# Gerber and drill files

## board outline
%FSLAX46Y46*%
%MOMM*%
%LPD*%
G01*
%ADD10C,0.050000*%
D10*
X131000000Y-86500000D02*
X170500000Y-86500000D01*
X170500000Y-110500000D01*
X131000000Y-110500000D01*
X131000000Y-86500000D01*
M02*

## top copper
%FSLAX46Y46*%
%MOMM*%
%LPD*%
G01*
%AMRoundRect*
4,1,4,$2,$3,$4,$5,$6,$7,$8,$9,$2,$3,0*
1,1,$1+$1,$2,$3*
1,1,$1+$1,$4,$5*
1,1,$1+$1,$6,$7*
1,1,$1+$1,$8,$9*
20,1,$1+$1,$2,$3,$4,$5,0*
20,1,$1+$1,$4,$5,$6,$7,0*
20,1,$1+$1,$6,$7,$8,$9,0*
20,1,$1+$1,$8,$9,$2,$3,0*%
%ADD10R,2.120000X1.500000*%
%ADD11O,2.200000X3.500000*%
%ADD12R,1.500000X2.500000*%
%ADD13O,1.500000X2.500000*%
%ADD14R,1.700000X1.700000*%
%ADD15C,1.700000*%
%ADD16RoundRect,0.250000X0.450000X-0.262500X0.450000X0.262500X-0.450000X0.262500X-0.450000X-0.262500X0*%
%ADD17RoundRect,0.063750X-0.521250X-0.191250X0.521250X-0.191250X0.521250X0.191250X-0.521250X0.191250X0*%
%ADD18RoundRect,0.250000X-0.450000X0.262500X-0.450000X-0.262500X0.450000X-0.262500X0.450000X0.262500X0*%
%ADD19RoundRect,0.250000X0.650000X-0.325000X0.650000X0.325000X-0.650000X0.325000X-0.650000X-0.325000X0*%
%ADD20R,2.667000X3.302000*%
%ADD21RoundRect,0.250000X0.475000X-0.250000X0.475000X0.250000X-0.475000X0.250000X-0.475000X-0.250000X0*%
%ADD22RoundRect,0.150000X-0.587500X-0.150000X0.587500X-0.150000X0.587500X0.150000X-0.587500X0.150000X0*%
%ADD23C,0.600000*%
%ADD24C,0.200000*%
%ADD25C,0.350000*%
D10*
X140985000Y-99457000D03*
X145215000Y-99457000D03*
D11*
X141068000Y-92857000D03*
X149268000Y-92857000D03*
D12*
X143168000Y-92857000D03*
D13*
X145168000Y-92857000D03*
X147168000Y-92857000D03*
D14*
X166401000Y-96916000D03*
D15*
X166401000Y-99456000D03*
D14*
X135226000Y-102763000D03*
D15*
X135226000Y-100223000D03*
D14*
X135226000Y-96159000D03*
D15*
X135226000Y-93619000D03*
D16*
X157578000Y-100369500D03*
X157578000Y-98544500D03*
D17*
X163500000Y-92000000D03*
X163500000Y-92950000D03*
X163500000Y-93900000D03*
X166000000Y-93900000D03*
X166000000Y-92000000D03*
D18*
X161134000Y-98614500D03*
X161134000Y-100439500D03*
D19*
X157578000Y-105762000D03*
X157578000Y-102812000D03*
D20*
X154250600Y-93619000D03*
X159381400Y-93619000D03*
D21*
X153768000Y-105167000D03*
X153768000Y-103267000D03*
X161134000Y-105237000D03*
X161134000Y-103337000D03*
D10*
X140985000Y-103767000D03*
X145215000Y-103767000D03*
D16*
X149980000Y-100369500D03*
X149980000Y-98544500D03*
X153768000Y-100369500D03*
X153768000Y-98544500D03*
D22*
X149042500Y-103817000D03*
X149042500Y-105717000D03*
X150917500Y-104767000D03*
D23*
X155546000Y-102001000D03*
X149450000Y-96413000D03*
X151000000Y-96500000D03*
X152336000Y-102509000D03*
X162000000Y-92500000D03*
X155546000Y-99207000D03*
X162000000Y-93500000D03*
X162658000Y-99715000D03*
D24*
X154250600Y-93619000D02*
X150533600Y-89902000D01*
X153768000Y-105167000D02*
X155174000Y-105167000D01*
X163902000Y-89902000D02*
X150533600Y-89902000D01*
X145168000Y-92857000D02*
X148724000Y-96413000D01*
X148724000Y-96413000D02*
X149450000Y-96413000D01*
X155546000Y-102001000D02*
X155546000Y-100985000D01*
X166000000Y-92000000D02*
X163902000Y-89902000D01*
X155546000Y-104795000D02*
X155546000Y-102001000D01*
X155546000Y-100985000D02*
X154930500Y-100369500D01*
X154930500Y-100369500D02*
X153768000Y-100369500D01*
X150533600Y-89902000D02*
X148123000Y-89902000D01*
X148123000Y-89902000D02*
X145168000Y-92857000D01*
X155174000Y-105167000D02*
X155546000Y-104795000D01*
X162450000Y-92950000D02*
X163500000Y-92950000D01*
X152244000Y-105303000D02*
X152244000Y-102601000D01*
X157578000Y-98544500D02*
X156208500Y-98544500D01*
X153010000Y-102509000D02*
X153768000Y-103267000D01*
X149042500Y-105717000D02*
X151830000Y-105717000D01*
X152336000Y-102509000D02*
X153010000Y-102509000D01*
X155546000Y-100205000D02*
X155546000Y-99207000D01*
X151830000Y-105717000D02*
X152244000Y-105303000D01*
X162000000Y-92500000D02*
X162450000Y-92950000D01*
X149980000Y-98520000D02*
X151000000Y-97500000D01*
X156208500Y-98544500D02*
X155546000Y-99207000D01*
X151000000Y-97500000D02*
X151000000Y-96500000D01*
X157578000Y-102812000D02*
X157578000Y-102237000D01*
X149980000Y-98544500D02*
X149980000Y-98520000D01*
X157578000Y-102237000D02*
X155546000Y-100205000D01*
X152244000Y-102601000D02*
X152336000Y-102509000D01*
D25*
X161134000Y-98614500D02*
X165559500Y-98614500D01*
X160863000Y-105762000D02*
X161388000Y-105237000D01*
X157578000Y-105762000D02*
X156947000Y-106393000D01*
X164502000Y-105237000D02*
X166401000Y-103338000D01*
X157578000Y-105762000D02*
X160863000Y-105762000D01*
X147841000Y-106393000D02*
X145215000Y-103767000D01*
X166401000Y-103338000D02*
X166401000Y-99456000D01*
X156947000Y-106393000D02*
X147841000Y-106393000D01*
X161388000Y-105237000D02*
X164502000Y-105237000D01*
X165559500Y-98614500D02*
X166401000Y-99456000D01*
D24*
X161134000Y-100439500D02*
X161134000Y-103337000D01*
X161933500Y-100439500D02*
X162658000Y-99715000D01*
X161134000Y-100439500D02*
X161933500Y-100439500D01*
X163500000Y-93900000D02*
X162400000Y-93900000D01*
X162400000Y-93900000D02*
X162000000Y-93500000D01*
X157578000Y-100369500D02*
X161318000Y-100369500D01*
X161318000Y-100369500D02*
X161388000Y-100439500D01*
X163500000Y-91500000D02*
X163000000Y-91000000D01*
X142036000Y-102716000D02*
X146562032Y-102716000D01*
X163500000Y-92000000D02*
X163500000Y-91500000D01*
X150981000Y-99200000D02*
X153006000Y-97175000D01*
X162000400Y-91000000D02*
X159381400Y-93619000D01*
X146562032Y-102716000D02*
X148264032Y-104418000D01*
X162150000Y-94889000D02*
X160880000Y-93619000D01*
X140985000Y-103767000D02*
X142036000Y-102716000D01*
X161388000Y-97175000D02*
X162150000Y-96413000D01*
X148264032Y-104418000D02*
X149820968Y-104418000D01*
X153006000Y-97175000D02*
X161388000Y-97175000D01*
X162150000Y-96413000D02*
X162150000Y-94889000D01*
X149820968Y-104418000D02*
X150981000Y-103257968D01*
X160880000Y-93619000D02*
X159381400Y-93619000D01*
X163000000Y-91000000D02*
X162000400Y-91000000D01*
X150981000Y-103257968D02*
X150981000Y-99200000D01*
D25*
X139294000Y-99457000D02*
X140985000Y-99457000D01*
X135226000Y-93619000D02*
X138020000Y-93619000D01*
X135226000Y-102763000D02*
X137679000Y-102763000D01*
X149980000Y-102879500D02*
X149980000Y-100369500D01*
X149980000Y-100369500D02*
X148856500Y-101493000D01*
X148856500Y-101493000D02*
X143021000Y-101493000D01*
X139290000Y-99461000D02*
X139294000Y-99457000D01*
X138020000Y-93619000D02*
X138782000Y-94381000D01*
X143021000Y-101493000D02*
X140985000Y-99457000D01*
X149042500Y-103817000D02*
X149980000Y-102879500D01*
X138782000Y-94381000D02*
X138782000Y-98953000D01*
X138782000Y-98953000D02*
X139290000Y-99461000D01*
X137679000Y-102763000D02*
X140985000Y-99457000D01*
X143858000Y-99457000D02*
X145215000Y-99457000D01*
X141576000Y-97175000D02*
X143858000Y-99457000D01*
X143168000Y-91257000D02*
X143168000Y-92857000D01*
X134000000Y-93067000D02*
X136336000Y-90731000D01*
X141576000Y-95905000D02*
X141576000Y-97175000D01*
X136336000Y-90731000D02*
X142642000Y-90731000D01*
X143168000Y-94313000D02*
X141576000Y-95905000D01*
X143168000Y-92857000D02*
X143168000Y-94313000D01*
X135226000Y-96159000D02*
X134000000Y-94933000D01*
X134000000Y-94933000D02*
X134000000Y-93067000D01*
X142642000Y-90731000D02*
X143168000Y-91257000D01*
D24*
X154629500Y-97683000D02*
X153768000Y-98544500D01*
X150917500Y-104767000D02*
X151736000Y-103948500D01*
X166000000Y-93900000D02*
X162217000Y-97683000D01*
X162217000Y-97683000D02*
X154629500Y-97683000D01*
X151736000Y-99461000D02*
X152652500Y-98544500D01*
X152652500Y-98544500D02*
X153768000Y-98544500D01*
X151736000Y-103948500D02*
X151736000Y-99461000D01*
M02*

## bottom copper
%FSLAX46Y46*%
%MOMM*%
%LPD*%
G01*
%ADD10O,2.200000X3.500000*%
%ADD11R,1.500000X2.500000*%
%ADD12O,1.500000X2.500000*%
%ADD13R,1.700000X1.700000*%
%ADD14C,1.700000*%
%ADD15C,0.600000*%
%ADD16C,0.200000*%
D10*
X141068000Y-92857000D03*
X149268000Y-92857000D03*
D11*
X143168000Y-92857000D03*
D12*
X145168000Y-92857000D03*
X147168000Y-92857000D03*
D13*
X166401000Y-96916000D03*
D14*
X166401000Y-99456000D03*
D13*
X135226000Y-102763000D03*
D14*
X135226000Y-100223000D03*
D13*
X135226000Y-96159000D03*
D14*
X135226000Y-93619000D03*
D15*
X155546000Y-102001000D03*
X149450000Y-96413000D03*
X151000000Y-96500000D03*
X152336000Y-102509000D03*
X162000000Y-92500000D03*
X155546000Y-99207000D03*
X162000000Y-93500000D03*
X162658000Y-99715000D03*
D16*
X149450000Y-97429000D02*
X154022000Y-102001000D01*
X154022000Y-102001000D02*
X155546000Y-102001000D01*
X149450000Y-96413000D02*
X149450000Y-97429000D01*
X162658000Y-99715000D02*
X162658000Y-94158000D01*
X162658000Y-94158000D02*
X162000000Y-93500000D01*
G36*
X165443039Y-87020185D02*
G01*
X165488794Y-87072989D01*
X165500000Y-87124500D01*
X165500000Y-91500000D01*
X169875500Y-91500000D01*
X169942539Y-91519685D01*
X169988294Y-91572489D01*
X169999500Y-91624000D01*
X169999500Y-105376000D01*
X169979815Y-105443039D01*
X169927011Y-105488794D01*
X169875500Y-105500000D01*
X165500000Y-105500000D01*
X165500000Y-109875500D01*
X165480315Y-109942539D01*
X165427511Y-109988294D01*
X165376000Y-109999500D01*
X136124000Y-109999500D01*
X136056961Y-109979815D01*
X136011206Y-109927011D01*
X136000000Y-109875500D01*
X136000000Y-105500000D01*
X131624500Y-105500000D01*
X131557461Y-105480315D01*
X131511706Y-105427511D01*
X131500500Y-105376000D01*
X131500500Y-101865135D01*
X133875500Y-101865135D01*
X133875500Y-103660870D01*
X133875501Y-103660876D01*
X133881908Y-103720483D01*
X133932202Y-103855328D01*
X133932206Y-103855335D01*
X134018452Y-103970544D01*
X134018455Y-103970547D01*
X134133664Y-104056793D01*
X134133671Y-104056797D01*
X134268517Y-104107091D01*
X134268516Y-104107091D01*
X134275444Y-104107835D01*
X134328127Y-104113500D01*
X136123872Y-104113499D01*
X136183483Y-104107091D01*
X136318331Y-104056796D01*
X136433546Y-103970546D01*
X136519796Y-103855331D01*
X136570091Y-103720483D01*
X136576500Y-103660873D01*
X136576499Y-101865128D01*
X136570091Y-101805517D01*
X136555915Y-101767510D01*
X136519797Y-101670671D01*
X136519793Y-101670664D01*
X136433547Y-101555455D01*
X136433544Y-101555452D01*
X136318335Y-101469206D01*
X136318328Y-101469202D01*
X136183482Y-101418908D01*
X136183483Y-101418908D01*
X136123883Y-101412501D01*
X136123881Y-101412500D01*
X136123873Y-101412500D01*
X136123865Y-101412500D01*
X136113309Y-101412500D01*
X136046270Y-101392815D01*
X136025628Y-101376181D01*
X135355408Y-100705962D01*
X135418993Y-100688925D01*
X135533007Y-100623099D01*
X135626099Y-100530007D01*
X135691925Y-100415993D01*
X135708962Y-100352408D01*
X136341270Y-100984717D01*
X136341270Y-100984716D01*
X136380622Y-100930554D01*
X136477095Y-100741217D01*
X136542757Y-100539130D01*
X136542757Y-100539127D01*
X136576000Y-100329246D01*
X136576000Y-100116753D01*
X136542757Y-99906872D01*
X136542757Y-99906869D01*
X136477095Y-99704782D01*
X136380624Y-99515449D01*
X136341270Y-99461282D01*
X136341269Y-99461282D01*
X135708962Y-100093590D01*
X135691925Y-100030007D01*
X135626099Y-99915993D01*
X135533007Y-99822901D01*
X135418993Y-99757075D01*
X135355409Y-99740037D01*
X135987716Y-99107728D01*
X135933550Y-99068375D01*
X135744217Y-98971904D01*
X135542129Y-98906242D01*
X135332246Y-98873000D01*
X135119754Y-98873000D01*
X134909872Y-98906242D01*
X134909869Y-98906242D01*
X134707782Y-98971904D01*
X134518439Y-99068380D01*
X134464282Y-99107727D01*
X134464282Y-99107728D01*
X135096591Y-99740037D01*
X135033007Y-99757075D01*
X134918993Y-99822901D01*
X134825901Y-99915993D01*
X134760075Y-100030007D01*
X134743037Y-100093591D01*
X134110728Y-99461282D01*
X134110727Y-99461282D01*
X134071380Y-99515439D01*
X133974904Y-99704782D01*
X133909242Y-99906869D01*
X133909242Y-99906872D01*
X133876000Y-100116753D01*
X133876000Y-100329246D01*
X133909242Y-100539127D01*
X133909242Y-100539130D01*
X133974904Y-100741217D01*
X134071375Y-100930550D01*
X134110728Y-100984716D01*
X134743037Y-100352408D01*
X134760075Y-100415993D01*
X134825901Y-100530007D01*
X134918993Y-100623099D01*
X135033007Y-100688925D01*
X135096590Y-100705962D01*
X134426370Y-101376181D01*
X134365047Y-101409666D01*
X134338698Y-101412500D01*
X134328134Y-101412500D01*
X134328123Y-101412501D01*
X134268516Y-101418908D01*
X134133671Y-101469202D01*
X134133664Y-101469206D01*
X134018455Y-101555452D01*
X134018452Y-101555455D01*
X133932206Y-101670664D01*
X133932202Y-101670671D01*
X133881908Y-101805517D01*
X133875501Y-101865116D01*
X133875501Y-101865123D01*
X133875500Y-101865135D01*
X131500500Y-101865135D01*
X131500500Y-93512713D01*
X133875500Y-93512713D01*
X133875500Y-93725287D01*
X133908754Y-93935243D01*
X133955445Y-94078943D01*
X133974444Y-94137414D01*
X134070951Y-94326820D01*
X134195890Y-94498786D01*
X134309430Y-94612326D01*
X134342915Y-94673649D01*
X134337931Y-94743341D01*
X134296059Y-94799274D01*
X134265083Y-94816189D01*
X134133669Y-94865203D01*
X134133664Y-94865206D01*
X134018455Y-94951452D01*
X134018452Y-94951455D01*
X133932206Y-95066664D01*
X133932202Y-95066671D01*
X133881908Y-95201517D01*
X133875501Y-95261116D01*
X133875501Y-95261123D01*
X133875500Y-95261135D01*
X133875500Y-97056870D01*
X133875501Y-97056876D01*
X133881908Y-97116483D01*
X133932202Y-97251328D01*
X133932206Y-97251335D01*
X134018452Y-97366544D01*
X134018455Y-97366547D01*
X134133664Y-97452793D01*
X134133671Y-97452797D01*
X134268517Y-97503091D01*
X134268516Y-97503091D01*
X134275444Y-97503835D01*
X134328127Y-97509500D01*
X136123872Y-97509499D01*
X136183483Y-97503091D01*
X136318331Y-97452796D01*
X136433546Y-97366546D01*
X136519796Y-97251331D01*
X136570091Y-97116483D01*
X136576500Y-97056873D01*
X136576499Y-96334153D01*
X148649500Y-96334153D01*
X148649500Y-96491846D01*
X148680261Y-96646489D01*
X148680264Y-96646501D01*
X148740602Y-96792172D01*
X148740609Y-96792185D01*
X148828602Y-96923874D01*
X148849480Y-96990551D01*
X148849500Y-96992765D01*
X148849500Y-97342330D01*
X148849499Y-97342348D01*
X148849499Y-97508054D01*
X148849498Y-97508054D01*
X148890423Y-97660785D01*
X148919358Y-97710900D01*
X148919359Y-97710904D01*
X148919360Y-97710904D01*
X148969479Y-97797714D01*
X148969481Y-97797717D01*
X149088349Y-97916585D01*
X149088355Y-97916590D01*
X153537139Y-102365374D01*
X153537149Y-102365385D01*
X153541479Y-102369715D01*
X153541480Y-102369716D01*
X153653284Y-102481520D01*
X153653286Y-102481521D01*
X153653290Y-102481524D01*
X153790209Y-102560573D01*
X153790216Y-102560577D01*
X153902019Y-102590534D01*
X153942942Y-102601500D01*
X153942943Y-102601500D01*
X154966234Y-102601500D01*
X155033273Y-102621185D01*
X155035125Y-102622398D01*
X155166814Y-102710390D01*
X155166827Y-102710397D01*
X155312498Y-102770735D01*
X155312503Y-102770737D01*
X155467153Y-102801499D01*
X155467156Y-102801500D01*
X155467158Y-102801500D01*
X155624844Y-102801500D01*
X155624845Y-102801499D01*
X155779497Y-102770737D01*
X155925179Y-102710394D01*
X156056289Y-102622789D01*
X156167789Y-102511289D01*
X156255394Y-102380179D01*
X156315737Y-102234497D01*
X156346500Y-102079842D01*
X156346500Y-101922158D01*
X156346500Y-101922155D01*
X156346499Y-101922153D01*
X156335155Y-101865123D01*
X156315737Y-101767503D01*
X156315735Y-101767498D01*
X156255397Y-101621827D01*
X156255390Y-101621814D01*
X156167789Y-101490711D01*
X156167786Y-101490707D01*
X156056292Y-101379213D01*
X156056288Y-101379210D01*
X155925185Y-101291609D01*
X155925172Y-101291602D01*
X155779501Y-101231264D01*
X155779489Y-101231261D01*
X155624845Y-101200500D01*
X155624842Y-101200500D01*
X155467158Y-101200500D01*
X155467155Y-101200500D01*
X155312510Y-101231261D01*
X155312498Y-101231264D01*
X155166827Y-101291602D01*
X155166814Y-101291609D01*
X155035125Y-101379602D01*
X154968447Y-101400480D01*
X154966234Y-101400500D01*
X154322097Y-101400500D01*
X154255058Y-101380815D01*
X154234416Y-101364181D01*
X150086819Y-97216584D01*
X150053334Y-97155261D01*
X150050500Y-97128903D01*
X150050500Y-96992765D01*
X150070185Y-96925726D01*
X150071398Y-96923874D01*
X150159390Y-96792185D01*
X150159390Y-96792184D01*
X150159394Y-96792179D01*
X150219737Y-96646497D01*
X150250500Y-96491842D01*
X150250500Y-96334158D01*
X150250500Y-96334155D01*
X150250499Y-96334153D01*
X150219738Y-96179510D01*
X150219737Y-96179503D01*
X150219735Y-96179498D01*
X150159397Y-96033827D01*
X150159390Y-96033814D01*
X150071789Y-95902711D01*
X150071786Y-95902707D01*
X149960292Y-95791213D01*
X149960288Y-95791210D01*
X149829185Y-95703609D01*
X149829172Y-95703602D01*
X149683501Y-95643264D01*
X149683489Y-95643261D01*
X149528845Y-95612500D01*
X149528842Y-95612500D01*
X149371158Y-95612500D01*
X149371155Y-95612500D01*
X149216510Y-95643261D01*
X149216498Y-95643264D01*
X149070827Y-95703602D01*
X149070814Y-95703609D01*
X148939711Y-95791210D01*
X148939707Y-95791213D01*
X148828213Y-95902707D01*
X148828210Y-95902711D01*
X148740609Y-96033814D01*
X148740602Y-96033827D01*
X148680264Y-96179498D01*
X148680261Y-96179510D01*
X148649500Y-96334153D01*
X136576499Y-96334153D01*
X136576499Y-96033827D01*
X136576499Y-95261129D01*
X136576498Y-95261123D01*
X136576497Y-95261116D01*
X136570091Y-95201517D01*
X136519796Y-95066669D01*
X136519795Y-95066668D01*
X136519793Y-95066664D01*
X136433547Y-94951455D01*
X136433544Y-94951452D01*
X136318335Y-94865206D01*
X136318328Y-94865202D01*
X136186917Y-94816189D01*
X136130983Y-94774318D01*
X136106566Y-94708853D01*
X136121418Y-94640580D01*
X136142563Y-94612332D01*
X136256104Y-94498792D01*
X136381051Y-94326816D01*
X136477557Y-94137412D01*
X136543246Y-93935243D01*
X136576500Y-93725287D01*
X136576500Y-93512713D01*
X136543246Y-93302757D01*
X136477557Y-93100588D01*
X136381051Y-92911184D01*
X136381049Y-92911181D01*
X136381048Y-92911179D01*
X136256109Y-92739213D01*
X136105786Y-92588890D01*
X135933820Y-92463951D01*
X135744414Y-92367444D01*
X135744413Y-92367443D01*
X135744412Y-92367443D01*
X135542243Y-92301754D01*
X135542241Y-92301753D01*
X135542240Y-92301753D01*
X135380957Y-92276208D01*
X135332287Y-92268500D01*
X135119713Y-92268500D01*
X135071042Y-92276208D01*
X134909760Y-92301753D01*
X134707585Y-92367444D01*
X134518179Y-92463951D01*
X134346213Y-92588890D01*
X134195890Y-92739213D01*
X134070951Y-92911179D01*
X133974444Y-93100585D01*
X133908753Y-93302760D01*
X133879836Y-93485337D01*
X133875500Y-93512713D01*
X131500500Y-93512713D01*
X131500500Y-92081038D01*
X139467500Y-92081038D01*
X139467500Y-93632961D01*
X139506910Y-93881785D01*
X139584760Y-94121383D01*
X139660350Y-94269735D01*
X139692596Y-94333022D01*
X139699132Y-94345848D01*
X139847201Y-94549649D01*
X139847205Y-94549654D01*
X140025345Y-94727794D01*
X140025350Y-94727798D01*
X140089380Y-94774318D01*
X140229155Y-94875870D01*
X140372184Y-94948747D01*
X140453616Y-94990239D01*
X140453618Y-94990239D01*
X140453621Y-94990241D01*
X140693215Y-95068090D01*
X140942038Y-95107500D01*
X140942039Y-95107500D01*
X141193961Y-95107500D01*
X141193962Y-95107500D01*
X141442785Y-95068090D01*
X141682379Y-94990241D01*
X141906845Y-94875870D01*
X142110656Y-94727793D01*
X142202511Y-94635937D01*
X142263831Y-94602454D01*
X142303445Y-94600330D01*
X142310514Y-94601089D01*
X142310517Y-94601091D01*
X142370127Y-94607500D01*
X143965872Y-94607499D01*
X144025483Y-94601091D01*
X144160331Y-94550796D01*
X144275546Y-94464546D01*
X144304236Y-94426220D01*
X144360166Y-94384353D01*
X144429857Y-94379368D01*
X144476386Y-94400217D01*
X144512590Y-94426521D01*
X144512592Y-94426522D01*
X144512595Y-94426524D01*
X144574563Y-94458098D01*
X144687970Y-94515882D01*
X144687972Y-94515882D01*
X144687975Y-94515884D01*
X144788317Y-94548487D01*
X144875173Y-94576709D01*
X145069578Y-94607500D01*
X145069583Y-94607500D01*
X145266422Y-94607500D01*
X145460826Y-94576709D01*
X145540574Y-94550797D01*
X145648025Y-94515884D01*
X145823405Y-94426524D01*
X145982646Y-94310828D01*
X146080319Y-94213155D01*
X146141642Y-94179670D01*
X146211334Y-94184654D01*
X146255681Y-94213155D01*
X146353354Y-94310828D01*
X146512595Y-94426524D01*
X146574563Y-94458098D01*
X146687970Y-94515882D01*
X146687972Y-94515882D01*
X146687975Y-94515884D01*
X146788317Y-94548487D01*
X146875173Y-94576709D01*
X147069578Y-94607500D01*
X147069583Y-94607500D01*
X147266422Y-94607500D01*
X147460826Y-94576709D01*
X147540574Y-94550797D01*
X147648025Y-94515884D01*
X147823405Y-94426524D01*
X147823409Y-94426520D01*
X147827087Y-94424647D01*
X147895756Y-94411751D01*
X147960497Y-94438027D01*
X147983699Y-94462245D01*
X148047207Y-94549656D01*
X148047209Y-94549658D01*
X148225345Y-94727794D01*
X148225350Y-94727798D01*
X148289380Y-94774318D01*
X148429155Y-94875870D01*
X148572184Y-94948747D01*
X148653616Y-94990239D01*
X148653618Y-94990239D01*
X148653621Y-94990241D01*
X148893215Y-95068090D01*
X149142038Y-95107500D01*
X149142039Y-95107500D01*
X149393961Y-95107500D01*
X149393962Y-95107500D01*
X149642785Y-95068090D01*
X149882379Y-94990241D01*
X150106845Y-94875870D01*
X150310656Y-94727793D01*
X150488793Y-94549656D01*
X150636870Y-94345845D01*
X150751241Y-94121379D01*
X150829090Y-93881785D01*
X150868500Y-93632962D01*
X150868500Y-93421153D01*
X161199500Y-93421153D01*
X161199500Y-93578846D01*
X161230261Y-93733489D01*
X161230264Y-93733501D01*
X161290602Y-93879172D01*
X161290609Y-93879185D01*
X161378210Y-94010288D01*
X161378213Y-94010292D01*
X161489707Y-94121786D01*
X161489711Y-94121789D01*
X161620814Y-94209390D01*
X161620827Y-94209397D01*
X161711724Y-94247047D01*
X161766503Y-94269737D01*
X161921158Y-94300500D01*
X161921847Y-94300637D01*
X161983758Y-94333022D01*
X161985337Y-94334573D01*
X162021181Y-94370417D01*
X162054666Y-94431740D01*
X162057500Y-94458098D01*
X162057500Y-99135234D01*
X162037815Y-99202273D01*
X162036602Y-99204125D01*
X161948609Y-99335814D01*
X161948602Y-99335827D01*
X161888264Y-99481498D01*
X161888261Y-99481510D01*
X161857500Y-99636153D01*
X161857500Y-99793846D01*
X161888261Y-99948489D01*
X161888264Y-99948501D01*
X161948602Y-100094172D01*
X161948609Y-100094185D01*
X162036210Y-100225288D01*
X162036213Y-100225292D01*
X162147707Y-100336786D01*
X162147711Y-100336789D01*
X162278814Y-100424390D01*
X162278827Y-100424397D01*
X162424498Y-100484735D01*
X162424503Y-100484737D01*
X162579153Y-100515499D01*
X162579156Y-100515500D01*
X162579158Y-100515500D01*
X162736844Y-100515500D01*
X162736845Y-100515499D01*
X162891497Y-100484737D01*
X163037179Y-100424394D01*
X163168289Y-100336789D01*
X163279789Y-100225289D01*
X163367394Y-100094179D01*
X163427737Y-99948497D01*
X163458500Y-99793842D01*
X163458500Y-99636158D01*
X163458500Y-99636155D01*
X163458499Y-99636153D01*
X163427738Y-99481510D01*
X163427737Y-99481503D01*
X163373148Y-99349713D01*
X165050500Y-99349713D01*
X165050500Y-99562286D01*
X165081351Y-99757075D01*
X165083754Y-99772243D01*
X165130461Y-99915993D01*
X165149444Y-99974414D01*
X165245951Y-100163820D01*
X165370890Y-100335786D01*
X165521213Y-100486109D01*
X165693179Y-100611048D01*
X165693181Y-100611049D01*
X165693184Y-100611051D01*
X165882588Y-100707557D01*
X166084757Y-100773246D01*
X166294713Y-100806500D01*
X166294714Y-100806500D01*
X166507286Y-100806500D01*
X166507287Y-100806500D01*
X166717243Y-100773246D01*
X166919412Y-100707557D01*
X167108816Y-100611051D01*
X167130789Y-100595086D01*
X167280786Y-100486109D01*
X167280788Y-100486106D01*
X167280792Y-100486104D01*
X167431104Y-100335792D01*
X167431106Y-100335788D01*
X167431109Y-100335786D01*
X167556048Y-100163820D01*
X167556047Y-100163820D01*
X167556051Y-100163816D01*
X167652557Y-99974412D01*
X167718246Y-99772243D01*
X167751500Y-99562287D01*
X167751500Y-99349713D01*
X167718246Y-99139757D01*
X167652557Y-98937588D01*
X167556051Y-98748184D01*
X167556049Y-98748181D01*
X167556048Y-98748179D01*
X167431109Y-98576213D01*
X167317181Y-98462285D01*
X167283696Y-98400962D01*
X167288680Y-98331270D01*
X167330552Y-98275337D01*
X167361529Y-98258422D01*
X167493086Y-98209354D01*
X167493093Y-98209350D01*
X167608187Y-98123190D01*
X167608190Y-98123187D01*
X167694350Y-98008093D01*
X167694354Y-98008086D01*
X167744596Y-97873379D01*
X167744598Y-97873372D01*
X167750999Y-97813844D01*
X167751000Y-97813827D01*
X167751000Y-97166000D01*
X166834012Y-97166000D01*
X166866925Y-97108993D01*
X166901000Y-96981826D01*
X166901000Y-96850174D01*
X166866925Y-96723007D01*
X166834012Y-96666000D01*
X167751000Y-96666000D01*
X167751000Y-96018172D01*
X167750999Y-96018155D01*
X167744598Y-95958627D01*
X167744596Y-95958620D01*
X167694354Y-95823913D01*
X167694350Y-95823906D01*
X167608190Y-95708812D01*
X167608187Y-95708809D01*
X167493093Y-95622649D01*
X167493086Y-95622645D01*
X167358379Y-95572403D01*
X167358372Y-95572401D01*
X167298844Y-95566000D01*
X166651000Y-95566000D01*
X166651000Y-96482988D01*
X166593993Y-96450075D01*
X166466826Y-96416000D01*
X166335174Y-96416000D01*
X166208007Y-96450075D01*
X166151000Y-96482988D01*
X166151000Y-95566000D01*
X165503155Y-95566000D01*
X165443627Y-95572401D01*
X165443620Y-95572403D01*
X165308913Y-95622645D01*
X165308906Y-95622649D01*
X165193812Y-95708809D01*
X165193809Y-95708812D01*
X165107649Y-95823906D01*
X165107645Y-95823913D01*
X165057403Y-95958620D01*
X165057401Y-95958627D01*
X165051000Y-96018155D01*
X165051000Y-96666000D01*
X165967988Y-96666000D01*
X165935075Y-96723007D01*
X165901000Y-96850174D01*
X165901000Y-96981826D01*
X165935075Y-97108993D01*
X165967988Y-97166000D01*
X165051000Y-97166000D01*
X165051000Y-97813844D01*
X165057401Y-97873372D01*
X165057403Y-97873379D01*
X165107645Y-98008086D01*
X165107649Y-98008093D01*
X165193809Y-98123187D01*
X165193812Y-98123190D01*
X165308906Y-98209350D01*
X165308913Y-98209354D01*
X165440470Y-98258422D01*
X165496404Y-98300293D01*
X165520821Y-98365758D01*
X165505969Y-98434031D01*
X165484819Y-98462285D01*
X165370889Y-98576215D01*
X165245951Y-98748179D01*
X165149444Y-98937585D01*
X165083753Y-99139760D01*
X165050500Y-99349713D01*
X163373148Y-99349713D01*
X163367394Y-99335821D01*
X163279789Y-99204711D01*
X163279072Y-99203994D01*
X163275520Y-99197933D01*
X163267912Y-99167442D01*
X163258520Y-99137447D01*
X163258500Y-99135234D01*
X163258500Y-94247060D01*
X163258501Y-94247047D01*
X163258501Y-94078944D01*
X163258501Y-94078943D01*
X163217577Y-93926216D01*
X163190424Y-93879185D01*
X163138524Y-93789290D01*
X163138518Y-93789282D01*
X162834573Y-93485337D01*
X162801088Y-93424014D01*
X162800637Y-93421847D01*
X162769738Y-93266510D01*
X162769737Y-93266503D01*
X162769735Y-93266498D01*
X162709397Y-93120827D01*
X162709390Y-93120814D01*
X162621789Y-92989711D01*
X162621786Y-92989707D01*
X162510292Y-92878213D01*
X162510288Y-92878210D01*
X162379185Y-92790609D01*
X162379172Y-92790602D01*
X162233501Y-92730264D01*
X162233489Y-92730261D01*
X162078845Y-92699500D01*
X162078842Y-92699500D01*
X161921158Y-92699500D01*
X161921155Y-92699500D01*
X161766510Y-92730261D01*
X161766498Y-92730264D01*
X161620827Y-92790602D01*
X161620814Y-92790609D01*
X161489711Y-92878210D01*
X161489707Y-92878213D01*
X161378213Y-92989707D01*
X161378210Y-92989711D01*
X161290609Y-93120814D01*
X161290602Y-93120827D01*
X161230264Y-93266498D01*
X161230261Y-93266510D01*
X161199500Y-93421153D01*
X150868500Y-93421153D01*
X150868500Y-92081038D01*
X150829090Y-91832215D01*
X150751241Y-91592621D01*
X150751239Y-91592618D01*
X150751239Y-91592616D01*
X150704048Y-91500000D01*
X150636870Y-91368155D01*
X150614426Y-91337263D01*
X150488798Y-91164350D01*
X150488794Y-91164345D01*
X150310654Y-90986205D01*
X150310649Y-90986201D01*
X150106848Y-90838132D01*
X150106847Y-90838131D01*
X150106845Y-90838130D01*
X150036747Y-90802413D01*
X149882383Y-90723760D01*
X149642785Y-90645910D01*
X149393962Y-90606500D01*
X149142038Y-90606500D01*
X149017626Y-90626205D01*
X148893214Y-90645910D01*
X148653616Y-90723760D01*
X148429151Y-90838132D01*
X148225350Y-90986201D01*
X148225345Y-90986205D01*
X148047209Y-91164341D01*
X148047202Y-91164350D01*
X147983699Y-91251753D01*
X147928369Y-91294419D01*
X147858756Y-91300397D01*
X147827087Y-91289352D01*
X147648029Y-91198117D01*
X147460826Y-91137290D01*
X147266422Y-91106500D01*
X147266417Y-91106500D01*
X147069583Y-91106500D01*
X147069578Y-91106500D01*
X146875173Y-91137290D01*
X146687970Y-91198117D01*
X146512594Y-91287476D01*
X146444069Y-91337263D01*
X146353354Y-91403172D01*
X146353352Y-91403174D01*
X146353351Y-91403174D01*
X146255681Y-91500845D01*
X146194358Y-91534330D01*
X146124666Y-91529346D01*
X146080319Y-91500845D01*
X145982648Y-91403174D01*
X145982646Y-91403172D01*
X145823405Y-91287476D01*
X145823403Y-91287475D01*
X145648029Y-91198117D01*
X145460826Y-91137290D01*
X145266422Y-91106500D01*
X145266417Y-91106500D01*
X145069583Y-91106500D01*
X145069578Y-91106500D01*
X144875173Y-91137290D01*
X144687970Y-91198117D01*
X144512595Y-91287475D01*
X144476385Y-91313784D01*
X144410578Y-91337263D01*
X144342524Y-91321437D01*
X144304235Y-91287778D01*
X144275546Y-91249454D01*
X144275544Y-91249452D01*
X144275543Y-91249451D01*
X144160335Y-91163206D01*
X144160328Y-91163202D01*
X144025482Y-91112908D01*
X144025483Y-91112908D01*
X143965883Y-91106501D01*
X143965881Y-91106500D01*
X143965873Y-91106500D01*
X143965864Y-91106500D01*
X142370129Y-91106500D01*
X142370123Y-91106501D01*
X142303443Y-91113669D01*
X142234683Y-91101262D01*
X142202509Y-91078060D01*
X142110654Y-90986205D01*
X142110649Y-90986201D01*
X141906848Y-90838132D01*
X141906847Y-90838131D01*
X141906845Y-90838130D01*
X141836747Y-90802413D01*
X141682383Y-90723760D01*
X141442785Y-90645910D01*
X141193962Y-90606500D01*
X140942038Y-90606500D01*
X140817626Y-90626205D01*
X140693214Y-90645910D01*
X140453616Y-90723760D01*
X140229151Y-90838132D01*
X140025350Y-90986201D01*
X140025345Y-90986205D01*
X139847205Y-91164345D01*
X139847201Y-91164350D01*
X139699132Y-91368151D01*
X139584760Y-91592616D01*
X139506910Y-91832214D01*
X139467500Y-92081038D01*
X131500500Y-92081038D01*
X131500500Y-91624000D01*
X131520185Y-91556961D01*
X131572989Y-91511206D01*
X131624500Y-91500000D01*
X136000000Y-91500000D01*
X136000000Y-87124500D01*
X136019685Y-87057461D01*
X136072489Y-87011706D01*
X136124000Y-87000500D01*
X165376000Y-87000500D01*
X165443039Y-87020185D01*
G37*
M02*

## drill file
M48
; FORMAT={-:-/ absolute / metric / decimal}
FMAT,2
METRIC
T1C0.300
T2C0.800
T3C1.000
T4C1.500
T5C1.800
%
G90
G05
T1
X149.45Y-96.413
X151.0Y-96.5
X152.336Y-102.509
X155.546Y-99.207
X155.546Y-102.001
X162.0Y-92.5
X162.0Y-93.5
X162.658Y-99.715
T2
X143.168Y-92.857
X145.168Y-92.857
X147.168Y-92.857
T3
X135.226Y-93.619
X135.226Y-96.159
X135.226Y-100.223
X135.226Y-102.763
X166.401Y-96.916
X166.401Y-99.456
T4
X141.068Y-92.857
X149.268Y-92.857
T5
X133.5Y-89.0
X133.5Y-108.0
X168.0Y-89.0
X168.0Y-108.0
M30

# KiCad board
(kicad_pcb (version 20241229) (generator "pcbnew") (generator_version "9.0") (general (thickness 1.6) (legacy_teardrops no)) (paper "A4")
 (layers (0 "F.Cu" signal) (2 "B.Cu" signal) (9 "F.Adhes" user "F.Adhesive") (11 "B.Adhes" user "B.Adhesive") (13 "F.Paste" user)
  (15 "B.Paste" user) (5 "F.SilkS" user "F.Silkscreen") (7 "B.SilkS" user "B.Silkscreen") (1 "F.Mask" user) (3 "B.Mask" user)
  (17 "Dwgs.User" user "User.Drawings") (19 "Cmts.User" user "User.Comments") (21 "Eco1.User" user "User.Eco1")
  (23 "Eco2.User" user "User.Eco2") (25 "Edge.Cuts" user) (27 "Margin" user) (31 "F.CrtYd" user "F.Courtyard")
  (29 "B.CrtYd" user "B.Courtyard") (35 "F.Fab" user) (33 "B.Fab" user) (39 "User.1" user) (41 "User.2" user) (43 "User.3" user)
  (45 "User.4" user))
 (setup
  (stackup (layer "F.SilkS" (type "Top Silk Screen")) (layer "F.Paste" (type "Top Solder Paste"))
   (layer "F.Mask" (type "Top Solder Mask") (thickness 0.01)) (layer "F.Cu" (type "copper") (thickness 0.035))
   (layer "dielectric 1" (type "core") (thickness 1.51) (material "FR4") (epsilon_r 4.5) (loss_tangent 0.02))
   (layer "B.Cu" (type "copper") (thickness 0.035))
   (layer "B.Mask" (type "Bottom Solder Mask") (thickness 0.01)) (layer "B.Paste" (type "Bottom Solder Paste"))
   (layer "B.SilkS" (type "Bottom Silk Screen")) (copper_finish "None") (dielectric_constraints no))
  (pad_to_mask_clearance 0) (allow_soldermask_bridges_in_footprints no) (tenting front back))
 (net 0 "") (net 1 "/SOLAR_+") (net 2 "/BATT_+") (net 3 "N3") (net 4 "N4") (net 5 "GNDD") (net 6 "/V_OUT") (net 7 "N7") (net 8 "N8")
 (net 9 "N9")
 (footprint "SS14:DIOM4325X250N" (layer "F.Cu") (at 143.1 99.457 180)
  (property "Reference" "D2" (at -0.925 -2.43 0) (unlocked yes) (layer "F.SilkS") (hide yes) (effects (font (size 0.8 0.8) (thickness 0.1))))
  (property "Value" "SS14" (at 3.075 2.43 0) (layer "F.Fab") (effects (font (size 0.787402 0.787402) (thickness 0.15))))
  (pad "A" smd rect (at 2.115 0 180) (size 2.12 1.5) (layers "F.Cu" "F.Mask" "F.Paste") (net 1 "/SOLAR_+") (solder_mask_margin 0.102))
  (pad "C" smd rect (at -2.115 0 180) (size 2.12 1.5) (layers "F.Cu" "F.Mask" "F.Paste") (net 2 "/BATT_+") (solder_mask_margin 0.102)))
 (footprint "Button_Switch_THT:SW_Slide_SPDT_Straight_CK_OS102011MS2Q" (layer "F.Cu") (at 143.168 92.857)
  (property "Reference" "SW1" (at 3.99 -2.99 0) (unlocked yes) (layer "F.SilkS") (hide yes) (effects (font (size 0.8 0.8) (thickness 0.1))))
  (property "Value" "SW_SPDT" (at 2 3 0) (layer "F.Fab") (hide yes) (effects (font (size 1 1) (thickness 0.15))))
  (pad "" thru_hole oval (at -2.1 0) (size 2.2 3.5) (drill 1.5) (layers "*.Cu" "*.Mask") (remove_unused_layers no))
  (pad "" thru_hole oval (at 6.1 0) (size 2.2 3.5) (drill 1.5) (layers "*.Cu" "*.Mask") (remove_unused_layers no))
  (pad "1" thru_hole rect (at 0 0) (size 1.5 2.5) (drill 0.8) (layers "*.Cu" "*.Mask") (remove_unused_layers no) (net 2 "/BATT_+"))
  (pad "2" thru_hole oval (at 2 0) (size 1.5 2.5) (drill 0.8) (layers "*.Cu" "*.Mask") (remove_unused_layers no) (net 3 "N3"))
  (pad "3" thru_hole oval (at 4 0) (size 1.5 2.5) (drill 0.8) (layers "*.Cu" "*.Mask") (remove_unused_layers no) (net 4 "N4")))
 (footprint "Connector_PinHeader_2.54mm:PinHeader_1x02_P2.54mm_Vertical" (layer "F.Cu") (at 166.401 96.916)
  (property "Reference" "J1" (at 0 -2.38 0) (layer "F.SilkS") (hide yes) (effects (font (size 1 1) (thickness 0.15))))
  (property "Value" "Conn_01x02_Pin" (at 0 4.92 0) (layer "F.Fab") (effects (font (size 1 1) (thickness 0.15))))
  (pad "1" thru_hole rect (at 0 0) (size 1.7 1.7) (drill 1) (layers "*.Cu" "*.Mask") (remove_unused_layers no) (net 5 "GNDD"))
  (pad "2" thru_hole circle (at 0 2.54) (size 1.7 1.7) (drill 1) (layers "*.Cu" "*.Mask") (remove_unused_layers no) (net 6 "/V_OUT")))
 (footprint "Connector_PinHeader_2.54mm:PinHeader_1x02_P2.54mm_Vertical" (layer "F.Cu") (at 135.226 102.763 180)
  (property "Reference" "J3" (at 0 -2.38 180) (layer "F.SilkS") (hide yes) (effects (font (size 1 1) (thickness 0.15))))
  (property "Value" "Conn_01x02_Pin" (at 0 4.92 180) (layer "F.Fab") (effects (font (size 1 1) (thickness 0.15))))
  (pad "1" thru_hole rect (at 0 0 180) (size 1.7 1.7) (drill 1) (layers "*.Cu" "*.Mask") (remove_unused_layers no) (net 1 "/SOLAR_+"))
  (pad "2" thru_hole circle (at 0 2.54 180) (size 1.7 1.7) (drill 1) (layers "*.Cu" "*.Mask") (remove_unused_layers no) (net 5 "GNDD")))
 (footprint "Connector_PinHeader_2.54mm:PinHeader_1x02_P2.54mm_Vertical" (layer "F.Cu") (at 135.226 96.159 180)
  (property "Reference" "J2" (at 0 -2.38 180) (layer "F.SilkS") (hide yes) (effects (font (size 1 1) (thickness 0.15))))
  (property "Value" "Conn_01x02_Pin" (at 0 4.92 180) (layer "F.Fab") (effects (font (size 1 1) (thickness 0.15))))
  (pad "1" thru_hole rect (at 0 0 180) (size 1.7 1.7) (drill 1) (layers "*.Cu" "*.Mask") (remove_unused_layers no) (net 2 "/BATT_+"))
  (pad "2" thru_hole circle (at 0 2.54 180) (size 1.7 1.7) (drill 1) (layers "*.Cu" "*.Mask") (remove_unused_layers no) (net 1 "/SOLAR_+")))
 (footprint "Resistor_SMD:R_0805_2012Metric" (layer "F.Cu") (at 157.578 99.457 90)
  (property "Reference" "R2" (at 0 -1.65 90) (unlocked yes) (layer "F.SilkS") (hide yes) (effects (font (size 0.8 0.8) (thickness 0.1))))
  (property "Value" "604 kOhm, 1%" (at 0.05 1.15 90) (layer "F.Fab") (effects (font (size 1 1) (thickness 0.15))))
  (pad "1" smd roundrect (at -0.9125 0 90) (size 1.025 1.4) (layers "F.Cu" "F.Mask" "F.Paste") (roundrect_rratio 0.243902) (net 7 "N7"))
  (pad "2" smd roundrect (at 0.9125 0 90) (size 1.025 1.4) (layers "F.Cu" "F.Mask" "F.Paste") (roundrect_rratio 0.243902) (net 5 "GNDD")))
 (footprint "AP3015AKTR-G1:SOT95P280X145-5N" (layer "F.Cu") (at 164.75 92.95)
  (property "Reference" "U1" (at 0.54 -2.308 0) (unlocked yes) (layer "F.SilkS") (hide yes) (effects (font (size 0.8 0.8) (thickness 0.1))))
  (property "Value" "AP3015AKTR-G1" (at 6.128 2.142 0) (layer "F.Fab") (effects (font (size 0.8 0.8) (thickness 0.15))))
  (pad "1" smd roundrect (at -1.25 -0.95) (size 1.17 0.51) (layers "F.Cu" "F.Mask" "F.Paste") (roundrect_rratio 0.125) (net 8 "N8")
   (solder_mask_margin 0.102))
  (pad "2" smd roundrect (at -1.25 0) (size 1.17 0.51) (layers "F.Cu" "F.Mask" "F.Paste") (roundrect_rratio 0.125) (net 5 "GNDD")
   (solder_mask_margin 0.102))
  (pad "3" smd roundrect (at -1.25 0.95) (size 1.17 0.51) (layers "F.Cu" "F.Mask" "F.Paste") (roundrect_rratio 0.125) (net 7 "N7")
   (solder_mask_margin 0.102))
  (pad "4" smd roundrect (at 1.25 0.95) (size 1.17 0.51) (layers "F.Cu" "F.Mask" "F.Paste") (roundrect_rratio 0.125) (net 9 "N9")
   (solder_mask_margin 0.102))
  (pad "5" smd roundrect (at 1.25 -0.95) (size 1.17 0.51) (layers "F.Cu" "F.Mask" "F.Paste") (roundrect_rratio 0.125) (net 3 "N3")
   (solder_mask_margin 0.102)))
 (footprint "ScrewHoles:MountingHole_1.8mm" (layer "F.Cu") (at 133.5 89)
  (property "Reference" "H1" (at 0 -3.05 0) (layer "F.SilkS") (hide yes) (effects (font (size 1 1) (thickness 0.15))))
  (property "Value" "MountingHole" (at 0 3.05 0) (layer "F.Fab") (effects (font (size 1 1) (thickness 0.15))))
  (pad "" np_thru_hole circle (at 0 0) (size 1.8 1.8) (drill 1.8) (layers "*.Cu" "*.Mask")))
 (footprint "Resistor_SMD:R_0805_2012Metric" (layer "F.Cu") (at 161.134 99.527 -90)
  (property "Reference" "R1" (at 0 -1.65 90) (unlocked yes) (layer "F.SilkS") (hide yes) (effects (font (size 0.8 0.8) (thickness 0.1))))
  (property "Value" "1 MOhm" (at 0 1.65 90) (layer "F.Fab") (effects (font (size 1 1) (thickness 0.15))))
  (pad "1" smd roundrect (at -0.9125 0 270) (size 1.025 1.4) (layers "F.Cu" "F.Mask" "F.Paste") (roundrect_rratio 0.243902) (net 6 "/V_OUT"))
  (pad "2" smd roundrect (at 0.9125 0 270) (size 1.025 1.4) (layers "F.Cu" "F.Mask" "F.Paste") (roundrect_rratio 0.243902) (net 7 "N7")))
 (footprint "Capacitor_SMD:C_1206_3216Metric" (layer "F.Cu") (at 157.578 104.287 90)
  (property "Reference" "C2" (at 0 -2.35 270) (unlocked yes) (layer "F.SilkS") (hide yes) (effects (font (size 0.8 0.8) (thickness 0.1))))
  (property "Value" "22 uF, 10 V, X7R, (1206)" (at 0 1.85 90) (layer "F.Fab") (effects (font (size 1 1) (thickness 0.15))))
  (pad "1" smd roundrect (at -1.475 0 90) (size 1.15 1.8) (layers "F.Cu" "F.Mask" "F.Paste") (roundrect_rratio 0.217391) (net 6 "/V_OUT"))
  (pad "2" smd roundrect (at 1.475 0 90) (size 1.15 1.8) (layers "F.Cu" "F.Mask" "F.Paste") (roundrect_rratio 0.217391) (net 5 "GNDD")))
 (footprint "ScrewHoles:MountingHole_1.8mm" (layer "F.Cu") (at 168 108)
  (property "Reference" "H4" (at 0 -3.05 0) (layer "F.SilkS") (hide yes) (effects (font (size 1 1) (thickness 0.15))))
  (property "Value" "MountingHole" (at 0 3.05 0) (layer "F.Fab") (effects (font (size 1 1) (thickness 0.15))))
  (pad "" np_thru_hole circle (at 0 0) (size 1.8 1.8) (drill 1.8) (layers "*.Cu" "*.Mask")))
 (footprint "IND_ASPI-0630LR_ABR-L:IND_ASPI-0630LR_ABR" (layer "F.Cu") (at 156.816 93.619)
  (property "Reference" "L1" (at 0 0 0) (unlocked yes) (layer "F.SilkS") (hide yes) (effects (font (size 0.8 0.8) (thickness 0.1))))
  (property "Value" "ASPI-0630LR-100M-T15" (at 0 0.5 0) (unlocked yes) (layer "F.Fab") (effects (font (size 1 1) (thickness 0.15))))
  (pad "1" smd rect (at -2.5654 0 90) (size 3.302 2.667) (layers "F.Cu" "F.Mask" "F.Paste") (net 3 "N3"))
  (pad "2" smd rect (at 2.5654 0 90) (size 3.302 2.667) (layers "F.Cu" "F.Mask" "F.Paste") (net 8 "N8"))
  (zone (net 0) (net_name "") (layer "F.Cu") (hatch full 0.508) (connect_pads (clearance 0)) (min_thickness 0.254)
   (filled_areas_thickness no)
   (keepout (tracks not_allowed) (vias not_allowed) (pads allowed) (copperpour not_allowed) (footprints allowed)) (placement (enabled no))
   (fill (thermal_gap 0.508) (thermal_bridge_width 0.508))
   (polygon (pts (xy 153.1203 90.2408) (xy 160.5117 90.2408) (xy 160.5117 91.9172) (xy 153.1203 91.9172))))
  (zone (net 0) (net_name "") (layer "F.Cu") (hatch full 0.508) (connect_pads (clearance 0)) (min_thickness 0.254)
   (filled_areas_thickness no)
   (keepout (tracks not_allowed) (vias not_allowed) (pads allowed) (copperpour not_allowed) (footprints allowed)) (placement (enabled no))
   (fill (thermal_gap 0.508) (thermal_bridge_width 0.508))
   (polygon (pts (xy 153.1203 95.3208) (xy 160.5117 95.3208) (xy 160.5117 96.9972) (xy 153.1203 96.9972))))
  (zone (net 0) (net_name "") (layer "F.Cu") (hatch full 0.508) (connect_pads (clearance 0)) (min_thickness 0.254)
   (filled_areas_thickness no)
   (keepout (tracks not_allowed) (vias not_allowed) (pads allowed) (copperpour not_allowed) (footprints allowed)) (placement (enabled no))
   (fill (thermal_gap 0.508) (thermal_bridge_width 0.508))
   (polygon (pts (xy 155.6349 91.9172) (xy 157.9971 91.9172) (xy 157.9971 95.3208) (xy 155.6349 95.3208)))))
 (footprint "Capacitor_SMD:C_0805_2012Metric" (layer "F.Cu") (at 153.768 104.217 90)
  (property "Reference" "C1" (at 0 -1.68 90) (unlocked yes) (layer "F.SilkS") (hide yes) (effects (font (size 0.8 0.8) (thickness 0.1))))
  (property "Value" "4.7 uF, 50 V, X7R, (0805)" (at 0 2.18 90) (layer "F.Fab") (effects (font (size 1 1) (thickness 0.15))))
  (pad "1" smd roundrect (at -0.95 0 90) (size 1 1.45) (layers "F.Cu" "F.Mask" "F.Paste") (roundrect_rratio 0.25) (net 3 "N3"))
  (pad "2" smd roundrect (at 0.95 0 90) (size 1 1.45) (layers "F.Cu" "F.Mask" "F.Paste") (roundrect_rratio 0.25) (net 5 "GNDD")))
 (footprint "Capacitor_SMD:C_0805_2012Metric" (layer "F.Cu") (at 161.134 104.287 90)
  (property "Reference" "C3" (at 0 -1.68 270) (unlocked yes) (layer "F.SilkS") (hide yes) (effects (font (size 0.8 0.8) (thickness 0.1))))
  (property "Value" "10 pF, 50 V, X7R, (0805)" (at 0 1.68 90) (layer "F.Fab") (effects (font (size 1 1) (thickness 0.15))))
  (pad "1" smd roundrect (at -0.95 0 90) (size 1 1.45) (layers "F.Cu" "F.Mask" "F.Paste") (roundrect_rratio 0.25) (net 6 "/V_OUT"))
  (pad "2" smd roundrect (at 0.95 0 90) (size 1 1.45) (layers "F.Cu" "F.Mask" "F.Paste") (roundrect_rratio 0.25) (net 7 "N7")))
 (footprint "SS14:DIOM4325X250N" (layer "F.Cu") (at 143.1 103.767 180)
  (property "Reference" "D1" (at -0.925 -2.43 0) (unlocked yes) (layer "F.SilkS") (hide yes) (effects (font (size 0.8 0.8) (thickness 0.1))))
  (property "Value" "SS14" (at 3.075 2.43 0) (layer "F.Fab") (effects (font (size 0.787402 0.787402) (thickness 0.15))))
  (pad "A" smd rect (at 2.115 0 180) (size 2.12 1.5) (layers "F.Cu" "F.Mask" "F.Paste") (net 8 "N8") (solder_mask_margin 0.102))
  (pad "C" smd rect (at -2.115 0 180) (size 2.12 1.5) (layers "F.Cu" "F.Mask" "F.Paste") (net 6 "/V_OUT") (solder_mask_margin 0.102)))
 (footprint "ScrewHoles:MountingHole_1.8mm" (layer "F.Cu") (at 133.5 108)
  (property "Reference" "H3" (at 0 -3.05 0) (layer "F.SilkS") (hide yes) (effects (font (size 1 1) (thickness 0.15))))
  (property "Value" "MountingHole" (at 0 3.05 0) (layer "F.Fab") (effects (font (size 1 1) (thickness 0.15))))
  (pad "" np_thru_hole circle (at 0 0) (size 1.8 1.8) (drill 1.8) (layers "*.Cu" "*.Mask")))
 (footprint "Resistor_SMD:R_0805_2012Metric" (layer "F.Cu") (at 149.98 99.457 90)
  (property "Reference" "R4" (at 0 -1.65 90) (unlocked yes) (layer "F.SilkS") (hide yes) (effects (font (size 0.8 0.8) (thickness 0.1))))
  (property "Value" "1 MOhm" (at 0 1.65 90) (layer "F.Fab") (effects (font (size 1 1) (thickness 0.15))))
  (pad "1" smd roundrect (at -0.9125 0 90) (size 1.025 1.4) (layers "F.Cu" "F.Mask" "F.Paste") (roundrect_rratio 0.243902)
   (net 1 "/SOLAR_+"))
  (pad "2" smd roundrect (at 0.9125 0 90) (size 1.025 1.4) (layers "F.Cu" "F.Mask" "F.Paste") (roundrect_rratio 0.243902) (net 5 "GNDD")))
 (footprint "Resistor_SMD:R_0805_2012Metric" (layer "F.Cu") (at 153.768 99.457 90)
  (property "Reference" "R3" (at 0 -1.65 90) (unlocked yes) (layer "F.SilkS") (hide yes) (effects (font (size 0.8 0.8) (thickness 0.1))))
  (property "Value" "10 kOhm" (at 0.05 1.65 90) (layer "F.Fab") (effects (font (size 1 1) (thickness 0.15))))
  (pad "1" smd roundrect (at -0.9125 0 90) (size 1.025 1.4) (layers "F.Cu" "F.Mask" "F.Paste") (roundrect_rratio 0.243902) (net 3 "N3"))
  (pad "2" smd roundrect (at 0.9125 0 90) (size 1.025 1.4) (layers "F.Cu" "F.Mask" "F.Paste") (roundrect_rratio 0.243902) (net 9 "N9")))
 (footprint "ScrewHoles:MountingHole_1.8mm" (layer "F.Cu") (at 168 89)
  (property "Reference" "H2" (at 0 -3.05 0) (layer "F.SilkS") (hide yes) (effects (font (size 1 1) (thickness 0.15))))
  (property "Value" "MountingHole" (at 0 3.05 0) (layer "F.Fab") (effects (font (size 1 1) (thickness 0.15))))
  (pad "" np_thru_hole circle (at 0 0) (size 1.8 1.8) (drill 1.8) (layers "*.Cu" "*.Mask")))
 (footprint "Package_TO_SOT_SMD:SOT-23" (layer "F.Cu") (at 149.98 104.767)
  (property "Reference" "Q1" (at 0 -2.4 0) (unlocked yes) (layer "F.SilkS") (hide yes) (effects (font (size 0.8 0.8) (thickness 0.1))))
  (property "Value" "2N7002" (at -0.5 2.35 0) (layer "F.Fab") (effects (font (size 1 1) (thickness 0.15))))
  (pad "1" smd roundrect (at -0.9375 -0.95) (size 1.475 0.6) (layers "F.Cu" "F.Mask" "F.Paste") (roundrect_rratio 0.25) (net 1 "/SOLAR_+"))
  (pad "2" smd roundrect (at -0.9375 0.95) (size 1.475 0.6) (layers "F.Cu" "F.Mask" "F.Paste") (roundrect_rratio 0.25) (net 5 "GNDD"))
  (pad "3" smd roundrect (at 0.9375 0) (size 1.475 0.6) (layers "F.Cu" "F.Mask" "F.Paste") (roundrect_rratio 0.25) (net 9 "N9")))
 (gr_rect (start 131 86.5) (end 170.5 110.5) (stroke (width 0.05) (type default)) (fill no) (layer "Edge.Cuts"))
 (segment (start 154.2506 93.619) (end 150.5336 89.902) (width 0.2) (layer "F.Cu") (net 3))
 (segment (start 153.768 105.167) (end 155.174 105.167) (width 0.2) (layer "F.Cu") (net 3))
 (segment (start 163.902 89.902) (end 150.5336 89.902) (width 0.2) (layer "F.Cu") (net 3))
 (segment (start 145.168 92.857) (end 148.724 96.413) (width 0.2) (layer "F.Cu") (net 3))
 (segment (start 148.724 96.413) (end 149.45 96.413) (width 0.2) (layer "F.Cu") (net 3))
 (segment (start 155.546 102.001) (end 155.546 100.985) (width 0.2) (layer "F.Cu") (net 3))
 (segment (start 166 92) (end 163.902 89.902) (width 0.2) (layer "F.Cu") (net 3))
 (segment (start 155.546 104.795) (end 155.546 102.001) (width 0.2) (layer "F.Cu") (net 3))
 (segment (start 155.546 100.985) (end 154.9305 100.3695) (width 0.2) (layer "F.Cu") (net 3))
 (segment (start 154.9305 100.3695) (end 153.768 100.3695) (width 0.2) (layer "F.Cu") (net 3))
 (segment (start 150.5336 89.902) (end 148.123 89.902) (width 0.2) (layer "F.Cu") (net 3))
 (segment (start 148.123 89.902) (end 145.168 92.857) (width 0.2) (layer "F.Cu") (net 3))
 (segment (start 155.174 105.167) (end 155.546 104.795) (width 0.2) (layer "F.Cu") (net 3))
 (via (at 155.546 102.001) (size 0.6) (drill 0.3) (layers "F.Cu" "B.Cu") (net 3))
 (via (at 149.45 96.413) (size 0.6) (drill 0.3) (layers "F.Cu" "B.Cu") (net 3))
 (segment (start 149.45 97.429) (end 154.022 102.001) (width 0.2) (layer "B.Cu") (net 3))
 (segment (start 154.022 102.001) (end 155.546 102.001) (width 0.2) (layer "B.Cu") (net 3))
 (segment (start 149.45 96.413) (end 149.45 97.429) (width 0.2) (layer "B.Cu") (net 3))
 (segment (start 162.45 92.95) (end 163.5 92.95) (width 0.2) (layer "F.Cu") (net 5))
 (segment (start 152.244 105.303) (end 152.244 102.601) (width 0.2) (layer "F.Cu") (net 5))
 (segment (start 157.578 98.5445) (end 156.2085 98.5445) (width 0.2) (layer "F.Cu") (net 5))
 (segment (start 153.01 102.509) (end 153.768 103.267) (width 0.2) (layer "F.Cu") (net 5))
 (segment (start 149.0425 105.717) (end 151.83 105.717) (width 0.2) (layer "F.Cu") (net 5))
 (segment (start 152.336 102.509) (end 153.01 102.509) (width 0.2) (layer "F.Cu") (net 5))
 (segment (start 155.546 100.205) (end 155.546 99.207) (width 0.2) (layer "F.Cu") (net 5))
 (segment (start 151.83 105.717) (end 152.244 105.303) (width 0.2) (layer "F.Cu") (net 5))
 (segment (start 162 92.5) (end 162.45 92.95) (width 0.2) (layer "F.Cu") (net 5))
 (segment (start 149.98 98.52) (end 151 97.5) (width 0.2) (layer "F.Cu") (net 5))
 (segment (start 156.2085 98.5445) (end 155.546 99.207) (width 0.2) (layer "F.Cu") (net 5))
 (segment (start 151 97.5) (end 151 96.5) (width 0.2) (layer "F.Cu") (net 5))
 (segment (start 157.578 102.812) (end 157.578 102.237) (width 0.2) (layer "F.Cu") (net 5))
 (segment (start 149.98 98.5445) (end 149.98 98.52) (width 0.2) (layer "F.Cu") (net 5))
 (segment (start 157.578 102.237) (end 155.546 100.205) (width 0.2) (layer "F.Cu") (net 5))
 (segment (start 152.244 102.601) (end 152.336 102.509) (width 0.2) (layer "F.Cu") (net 5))
 (via (at 151 96.5) (size 0.6) (drill 0.3) (layers "F.Cu" "B.Cu") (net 5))
 (via (at 152.336 102.509) (size 0.6) (drill 0.3) (layers "F.Cu" "B.Cu") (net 5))
 (via (at 162 92.5) (size 0.6) (drill 0.3) (layers "F.Cu" "B.Cu") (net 5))
 (via (at 155.546 99.207) (size 0.6) (drill 0.3) (layers "F.Cu" "B.Cu") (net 5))
 (segment (start 161.134 98.6145) (end 165.5595 98.6145) (width 0.35) (layer "F.Cu") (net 6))
 (segment (start 160.863 105.762) (end 161.388 105.237) (width 0.35) (layer "F.Cu") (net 6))
 (segment (start 157.578 105.762) (end 156.947 106.393) (width 0.35) (layer "F.Cu") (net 6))
 (segment (start 164.502 105.237) (end 166.401 103.338) (width 0.35) (layer "F.Cu") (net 6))
 (segment (start 157.578 105.762) (end 160.863 105.762) (width 0.35) (layer "F.Cu") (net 6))
 (segment (start 147.841 106.393) (end 145.215 103.767) (width 0.35) (layer "F.Cu") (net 6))
 (segment (start 166.401 103.338) (end 166.401 99.456) (width 0.35) (layer "F.Cu") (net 6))
 (segment (start 156.947 106.393) (end 147.841 106.393) (width 0.35) (layer "F.Cu") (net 6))
 (segment (start 161.388 105.237) (end 164.502 105.237) (width 0.35) (layer "F.Cu") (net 6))
 (segment (start 165.5595 98.6145) (end 166.401 99.456) (width 0.35) (layer "F.Cu") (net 6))
 (segment (start 161.134 100.4395) (end 161.134 103.337) (width 0.2) (layer "F.Cu") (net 7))
 (segment (start 161.9335 100.4395) (end 162.658 99.715) (width 0.2) (layer "F.Cu") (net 7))
 (segment (start 161.134 100.4395) (end 161.9335 100.4395) (width 0.2) (layer "F.Cu") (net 7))
 (segment (start 163.5 93.9) (end 162.4 93.9) (width 0.2) (layer "F.Cu") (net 7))
 (segment (start 162.4 93.9) (end 162 93.5) (width 0.2) (layer "F.Cu") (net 7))
 (segment (start 157.578 100.3695) (end 161.318 100.3695) (width 0.2) (layer "F.Cu") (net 7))
 (segment (start 161.318 100.3695) (end 161.388 100.4395) (width 0.2) (layer "F.Cu") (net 7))
 (via (at 162 93.5) (size 0.6) (drill 0.3) (layers "F.Cu" "B.Cu") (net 7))
 (via (at 162.658 99.715) (size 0.6) (drill 0.3) (layers "F.Cu" "B.Cu") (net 7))
 (segment (start 162.658 99.715) (end 162.658 94.158) (width 0.2) (layer "B.Cu") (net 7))
 (segment (start 162.658 94.158) (end 162 93.5) (width 0.2) (layer "B.Cu") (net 7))
 (segment (start 163.5 91.5) (end 163 91) (width 0.2) (layer "F.Cu") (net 8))
 (segment (start 142.036 102.716) (end 146.562032 102.716) (width 0.2) (layer "F.Cu") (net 8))
 (segment (start 163.5 92) (end 163.5 91.5) (width 0.2) (layer "F.Cu") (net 8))
 (segment (start 150.981 99.2) (end 153.006 97.175) (width 0.2) (layer "F.Cu") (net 8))
 (segment (start 162.0004 91) (end 159.3814 93.619) (width 0.2) (layer "F.Cu") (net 8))
 (segment (start 146.562032 102.716) (end 148.264032 104.418) (width 0.2) (layer "F.Cu") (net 8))
 (segment (start 162.15 94.889) (end 160.88 93.619) (width 0.2) (layer "F.Cu") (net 8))
 (segment (start 140.985 103.767) (end 142.036 102.716) (width 0.2) (layer "F.Cu") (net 8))
 (segment (start 161.388 97.175) (end 162.15 96.413) (width 0.2) (layer "F.Cu") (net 8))
 (segment (start 148.264032 104.418) (end 149.820968 104.418) (width 0.2) (layer "F.Cu") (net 8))
 (segment (start 153.006 97.175) (end 161.388 97.175) (width 0.2) (layer "F.Cu") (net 8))
 (segment (start 162.15 96.413) (end 162.15 94.889) (width 0.2) (layer "F.Cu") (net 8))
 (segment (start 149.820968 104.418) (end 150.981 103.257968) (width 0.2) (layer "F.Cu") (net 8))
 (segment (start 160.88 93.619) (end 159.3814 93.619) (width 0.2) (layer "F.Cu") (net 8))
 (segment (start 163 91) (end 162.0004 91) (width 0.2) (layer "F.Cu") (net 8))
 (segment (start 150.981 103.257968) (end 150.981 99.2) (width 0.2) (layer "F.Cu") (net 8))
 (segment (start 139.294 99.457) (end 140.985 99.457) (width 0.35) (layer "F.Cu") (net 1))
 (segment (start 135.226 93.619) (end 138.02 93.619) (width 0.35) (layer "F.Cu") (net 1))
 (segment (start 135.226 102.763) (end 137.679 102.763) (width 0.35) (layer "F.Cu") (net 1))
 (segment (start 149.98 102.8795) (end 149.98 100.3695) (width 0.35) (layer "F.Cu") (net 1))
 (segment (start 149.98 100.3695) (end 148.8565 101.493) (width 0.35) (layer "F.Cu") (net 1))
 (segment (start 148.8565 101.493) (end 143.021 101.493) (width 0.35) (layer "F.Cu") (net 1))
 (segment (start 139.29 99.461) (end 139.294 99.457) (width 0.35) (layer "F.Cu") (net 1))
 (segment (start 138.02 93.619) (end 138.782 94.381) (width 0.35) (layer "F.Cu") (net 1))
 (segment (start 143.021 101.493) (end 140.985 99.457) (width 0.35) (layer "F.Cu") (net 1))
 (segment (start 149.0425 103.817) (end 149.98 102.8795) (width 0.35) (layer "F.Cu") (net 1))
 (segment (start 138.782 94.381) (end 138.782 98.953) (width 0.35) (layer "F.Cu") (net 1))
 (segment (start 138.782 98.953) (end 139.29 99.461) (width 0.35) (layer "F.Cu") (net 1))
 (segment (start 137.679 102.763) (end 140.985 99.457) (width 0.35) (layer "F.Cu") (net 1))
 (segment (start 143.858 99.457) (end 145.215 99.457) (width 0.35) (layer "F.Cu") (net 2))
 (segment (start 141.576 97.175) (end 143.858 99.457) (width 0.35) (layer "F.Cu") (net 2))
 (segment (start 143.168 91.257) (end 143.168 92.857) (width 0.35) (layer "F.Cu") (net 2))
 (segment (start 134 93.067) (end 136.336 90.731) (width 0.35) (layer "F.Cu") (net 2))
 (segment (start 141.576 95.905) (end 141.576 97.175) (width 0.35) (layer "F.Cu") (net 2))
 (segment (start 136.336 90.731) (end 142.642 90.731) (width 0.35) (layer "F.Cu") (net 2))
 (segment (start 143.168 94.313) (end 141.576 95.905) (width 0.35) (layer "F.Cu") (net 2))
 (segment (start 143.168 92.857) (end 143.168 94.313) (width 0.35) (layer "F.Cu") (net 2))
 (segment (start 135.226 96.159) (end 134 94.933) (width 0.35) (layer "F.Cu") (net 2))
 (segment (start 134 94.933) (end 134 93.067) (width 0.35) (layer "F.Cu") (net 2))
 (segment (start 142.642 90.731) (end 143.168 91.257) (width 0.35) (layer "F.Cu") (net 2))
 (segment (start 154.6295 97.683) (end 153.768 98.5445) (width 0.2) (layer "F.Cu") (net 9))
 (segment (start 150.9175 104.767) (end 151.736 103.9485) (width 0.2) (layer "F.Cu") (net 9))
 (segment (start 166 93.9) (end 162.217 97.683) (width 0.2) (layer "F.Cu") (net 9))
 (segment (start 162.217 97.683) (end 154.6295 97.683) (width 0.2) (layer "F.Cu") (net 9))
 (segment (start 151.736 99.461) (end 152.6525 98.5445) (width 0.2) (layer "F.Cu") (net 9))
 (segment (start 152.6525 98.5445) (end 153.768 98.5445) (width 0.2) (layer "F.Cu") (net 9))
 (segment (start 151.736 103.9485) (end 151.736 99.461) (width 0.2) (layer "F.Cu") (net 9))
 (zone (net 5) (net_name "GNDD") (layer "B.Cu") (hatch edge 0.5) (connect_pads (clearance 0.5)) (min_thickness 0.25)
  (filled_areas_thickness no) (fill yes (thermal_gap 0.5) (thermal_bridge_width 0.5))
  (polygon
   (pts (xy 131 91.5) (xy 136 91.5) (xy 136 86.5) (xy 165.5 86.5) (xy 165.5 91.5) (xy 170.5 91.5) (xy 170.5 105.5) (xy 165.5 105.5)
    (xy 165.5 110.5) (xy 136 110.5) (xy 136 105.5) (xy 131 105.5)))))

